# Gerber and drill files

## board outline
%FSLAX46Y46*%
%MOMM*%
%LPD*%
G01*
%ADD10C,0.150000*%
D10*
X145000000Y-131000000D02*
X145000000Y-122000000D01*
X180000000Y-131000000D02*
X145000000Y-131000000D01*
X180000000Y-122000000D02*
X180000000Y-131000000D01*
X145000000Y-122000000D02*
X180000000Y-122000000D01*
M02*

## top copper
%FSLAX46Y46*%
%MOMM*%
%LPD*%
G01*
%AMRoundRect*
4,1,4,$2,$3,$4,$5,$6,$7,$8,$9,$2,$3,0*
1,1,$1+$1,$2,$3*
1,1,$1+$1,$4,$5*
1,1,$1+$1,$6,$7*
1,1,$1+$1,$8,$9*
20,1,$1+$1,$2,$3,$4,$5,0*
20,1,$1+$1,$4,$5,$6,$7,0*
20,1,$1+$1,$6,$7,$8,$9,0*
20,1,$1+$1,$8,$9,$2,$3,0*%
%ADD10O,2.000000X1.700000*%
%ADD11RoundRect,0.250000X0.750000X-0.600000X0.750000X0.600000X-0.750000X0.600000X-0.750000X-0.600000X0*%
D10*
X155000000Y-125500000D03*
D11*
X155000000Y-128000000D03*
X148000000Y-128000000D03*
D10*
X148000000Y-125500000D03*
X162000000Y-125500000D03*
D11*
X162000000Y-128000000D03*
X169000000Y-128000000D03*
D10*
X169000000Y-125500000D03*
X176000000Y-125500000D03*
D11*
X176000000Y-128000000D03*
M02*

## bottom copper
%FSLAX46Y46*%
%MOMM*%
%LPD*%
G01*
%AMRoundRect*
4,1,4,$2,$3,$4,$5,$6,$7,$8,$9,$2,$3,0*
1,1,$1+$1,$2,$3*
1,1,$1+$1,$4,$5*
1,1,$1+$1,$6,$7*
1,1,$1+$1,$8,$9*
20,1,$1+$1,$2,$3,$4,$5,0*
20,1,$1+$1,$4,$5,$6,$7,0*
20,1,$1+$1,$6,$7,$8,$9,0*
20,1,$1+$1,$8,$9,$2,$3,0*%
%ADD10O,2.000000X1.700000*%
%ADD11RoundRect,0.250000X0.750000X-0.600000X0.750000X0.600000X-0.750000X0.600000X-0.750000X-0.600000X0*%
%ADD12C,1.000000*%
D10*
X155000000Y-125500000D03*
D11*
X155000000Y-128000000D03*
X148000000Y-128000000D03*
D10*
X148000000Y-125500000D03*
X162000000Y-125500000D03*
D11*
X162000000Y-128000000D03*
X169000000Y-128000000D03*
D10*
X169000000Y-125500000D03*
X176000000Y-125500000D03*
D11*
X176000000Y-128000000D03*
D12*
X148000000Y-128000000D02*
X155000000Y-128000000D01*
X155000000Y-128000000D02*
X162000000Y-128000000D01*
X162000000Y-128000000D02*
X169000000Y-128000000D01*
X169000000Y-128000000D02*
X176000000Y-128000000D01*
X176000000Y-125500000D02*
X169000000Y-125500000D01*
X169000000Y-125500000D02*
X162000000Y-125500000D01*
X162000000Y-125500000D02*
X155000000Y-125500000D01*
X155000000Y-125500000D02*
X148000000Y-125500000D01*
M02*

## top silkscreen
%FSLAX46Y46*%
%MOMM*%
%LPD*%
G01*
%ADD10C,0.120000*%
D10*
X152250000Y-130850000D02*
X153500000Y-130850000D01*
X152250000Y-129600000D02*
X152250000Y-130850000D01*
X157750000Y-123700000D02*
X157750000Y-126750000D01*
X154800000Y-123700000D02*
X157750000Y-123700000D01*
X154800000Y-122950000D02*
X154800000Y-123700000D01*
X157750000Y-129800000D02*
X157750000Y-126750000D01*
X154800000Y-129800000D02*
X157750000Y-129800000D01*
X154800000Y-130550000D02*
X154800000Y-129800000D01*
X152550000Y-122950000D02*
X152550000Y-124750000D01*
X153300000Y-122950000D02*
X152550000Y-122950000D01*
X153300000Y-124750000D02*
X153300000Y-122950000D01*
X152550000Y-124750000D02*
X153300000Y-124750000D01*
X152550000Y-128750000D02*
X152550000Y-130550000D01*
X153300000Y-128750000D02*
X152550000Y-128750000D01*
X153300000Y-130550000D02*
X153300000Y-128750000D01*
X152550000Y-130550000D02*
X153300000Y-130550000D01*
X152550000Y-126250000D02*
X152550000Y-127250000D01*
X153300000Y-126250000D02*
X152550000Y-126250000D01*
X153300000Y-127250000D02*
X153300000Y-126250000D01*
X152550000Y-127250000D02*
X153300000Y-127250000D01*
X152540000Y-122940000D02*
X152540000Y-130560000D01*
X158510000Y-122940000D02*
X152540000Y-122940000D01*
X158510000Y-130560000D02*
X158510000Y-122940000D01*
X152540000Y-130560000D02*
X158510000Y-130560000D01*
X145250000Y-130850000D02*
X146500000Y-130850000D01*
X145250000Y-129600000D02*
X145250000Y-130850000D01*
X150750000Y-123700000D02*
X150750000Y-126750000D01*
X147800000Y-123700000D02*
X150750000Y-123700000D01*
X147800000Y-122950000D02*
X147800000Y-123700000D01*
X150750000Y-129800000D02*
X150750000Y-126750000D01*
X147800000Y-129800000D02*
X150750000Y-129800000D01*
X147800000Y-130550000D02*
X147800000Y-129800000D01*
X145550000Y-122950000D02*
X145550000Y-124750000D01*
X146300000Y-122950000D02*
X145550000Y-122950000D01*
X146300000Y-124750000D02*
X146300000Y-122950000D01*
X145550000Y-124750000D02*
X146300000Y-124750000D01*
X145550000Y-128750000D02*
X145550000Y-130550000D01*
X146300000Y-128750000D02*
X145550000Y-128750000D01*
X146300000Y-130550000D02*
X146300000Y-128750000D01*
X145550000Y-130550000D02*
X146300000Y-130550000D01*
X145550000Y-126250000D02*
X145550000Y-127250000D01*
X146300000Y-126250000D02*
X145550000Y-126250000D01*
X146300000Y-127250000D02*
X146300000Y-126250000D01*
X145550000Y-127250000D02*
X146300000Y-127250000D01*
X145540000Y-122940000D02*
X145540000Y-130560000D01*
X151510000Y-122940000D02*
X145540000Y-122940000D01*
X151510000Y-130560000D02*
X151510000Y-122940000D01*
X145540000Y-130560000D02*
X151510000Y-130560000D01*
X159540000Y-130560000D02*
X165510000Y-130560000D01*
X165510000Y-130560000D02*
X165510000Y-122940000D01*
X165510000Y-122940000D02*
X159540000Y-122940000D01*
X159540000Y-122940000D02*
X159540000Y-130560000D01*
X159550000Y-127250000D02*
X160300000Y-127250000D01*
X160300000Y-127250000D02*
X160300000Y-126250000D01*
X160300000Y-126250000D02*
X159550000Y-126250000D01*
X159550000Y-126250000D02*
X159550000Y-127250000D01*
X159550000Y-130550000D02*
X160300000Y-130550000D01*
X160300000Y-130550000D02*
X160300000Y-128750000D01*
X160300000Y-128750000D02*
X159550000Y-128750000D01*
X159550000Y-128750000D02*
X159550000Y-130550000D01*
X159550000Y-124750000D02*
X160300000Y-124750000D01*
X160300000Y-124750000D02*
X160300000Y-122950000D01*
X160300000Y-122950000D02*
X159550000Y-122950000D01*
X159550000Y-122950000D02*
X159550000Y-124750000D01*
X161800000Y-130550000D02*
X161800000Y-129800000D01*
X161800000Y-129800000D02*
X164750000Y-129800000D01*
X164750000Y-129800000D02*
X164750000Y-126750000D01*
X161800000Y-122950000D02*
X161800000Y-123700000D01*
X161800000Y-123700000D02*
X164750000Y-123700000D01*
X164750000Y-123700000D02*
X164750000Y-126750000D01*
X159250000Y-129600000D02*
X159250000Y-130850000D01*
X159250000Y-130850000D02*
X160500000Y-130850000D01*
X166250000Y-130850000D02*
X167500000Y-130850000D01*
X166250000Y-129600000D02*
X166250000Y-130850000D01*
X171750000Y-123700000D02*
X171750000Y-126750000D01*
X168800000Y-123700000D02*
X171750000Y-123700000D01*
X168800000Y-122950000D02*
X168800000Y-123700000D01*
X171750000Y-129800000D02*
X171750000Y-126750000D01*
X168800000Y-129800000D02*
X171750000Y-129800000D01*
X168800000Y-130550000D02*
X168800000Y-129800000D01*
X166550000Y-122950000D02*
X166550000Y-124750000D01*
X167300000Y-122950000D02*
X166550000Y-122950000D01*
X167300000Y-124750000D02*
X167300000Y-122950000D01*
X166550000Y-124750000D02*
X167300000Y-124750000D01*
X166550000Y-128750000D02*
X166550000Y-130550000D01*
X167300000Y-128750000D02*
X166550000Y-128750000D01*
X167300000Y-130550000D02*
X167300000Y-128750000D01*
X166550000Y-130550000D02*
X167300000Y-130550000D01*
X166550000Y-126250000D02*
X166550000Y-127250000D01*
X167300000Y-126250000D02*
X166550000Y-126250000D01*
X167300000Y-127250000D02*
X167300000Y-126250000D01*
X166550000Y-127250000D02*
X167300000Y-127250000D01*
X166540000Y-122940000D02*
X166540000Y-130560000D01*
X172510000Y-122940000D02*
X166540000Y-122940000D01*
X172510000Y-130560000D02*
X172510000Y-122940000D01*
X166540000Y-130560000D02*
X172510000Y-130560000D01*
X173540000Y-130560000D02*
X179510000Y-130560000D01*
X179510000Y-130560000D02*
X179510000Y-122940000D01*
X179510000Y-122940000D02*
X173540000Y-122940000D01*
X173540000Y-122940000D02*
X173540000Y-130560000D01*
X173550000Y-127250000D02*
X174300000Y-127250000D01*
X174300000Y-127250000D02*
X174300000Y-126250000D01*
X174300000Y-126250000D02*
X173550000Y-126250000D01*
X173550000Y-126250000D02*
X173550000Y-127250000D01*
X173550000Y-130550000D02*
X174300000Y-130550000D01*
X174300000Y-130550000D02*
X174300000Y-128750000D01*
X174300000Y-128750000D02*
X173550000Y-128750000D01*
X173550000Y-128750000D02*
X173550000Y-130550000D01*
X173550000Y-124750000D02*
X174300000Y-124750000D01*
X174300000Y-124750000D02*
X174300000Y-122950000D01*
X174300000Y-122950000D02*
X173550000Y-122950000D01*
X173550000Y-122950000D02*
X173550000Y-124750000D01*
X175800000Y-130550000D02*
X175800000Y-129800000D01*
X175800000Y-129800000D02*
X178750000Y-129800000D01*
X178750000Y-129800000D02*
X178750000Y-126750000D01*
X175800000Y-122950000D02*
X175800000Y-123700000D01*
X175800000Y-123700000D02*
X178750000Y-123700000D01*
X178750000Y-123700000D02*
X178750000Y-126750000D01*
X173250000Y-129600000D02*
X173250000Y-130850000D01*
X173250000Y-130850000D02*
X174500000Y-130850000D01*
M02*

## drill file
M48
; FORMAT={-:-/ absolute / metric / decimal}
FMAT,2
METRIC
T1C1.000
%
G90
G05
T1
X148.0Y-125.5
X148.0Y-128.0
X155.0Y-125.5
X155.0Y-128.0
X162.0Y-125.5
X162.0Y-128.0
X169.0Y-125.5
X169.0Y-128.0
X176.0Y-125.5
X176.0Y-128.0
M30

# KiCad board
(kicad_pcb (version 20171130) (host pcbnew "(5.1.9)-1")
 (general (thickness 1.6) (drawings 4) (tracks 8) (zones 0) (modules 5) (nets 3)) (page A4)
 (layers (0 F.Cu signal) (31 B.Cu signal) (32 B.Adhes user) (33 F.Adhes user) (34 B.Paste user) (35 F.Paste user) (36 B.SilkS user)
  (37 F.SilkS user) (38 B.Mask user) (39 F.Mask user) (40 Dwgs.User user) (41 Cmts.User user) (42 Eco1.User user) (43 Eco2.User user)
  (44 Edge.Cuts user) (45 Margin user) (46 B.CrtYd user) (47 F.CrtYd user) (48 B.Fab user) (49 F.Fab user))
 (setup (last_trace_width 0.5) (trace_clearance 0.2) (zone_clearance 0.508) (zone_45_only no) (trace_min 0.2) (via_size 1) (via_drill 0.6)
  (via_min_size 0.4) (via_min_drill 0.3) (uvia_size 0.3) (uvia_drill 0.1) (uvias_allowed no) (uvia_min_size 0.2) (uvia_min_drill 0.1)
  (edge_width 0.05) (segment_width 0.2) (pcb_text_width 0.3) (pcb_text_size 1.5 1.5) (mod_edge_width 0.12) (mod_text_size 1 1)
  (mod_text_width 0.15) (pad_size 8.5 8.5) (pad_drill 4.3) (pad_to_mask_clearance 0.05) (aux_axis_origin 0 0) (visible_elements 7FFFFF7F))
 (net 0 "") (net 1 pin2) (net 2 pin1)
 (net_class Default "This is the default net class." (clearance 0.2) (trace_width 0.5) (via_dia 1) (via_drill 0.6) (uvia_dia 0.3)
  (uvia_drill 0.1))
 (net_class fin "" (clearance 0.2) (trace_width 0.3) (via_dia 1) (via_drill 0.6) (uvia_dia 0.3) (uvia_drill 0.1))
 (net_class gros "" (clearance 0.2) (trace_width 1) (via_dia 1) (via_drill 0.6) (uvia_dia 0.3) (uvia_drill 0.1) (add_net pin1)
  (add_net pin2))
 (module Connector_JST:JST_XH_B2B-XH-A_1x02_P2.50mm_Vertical (layer F.Cu) (at 155 128 90)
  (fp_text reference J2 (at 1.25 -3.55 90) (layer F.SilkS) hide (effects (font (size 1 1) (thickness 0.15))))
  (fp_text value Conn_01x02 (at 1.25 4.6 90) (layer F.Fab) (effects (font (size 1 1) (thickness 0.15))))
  (fp_line (start -2.85 -2.75) (end -2.85 -1.5) (layer F.SilkS) (width 0.12))
  (fp_line (start -1.6 -2.75) (end -2.85 -2.75) (layer F.SilkS) (width 0.12))
  (fp_line (start 4.3 2.75) (end 1.25 2.75) (layer F.SilkS) (width 0.12))
  (fp_line (start 4.3 -0.2) (end 4.3 2.75) (layer F.SilkS) (width 0.12))
  (fp_line (start 5.05 -0.2) (end 4.3 -0.2) (layer F.SilkS) (width 0.12))
  (fp_line (start -1.8 2.75) (end 1.25 2.75) (layer F.SilkS) (width 0.12))
  (fp_line (start -1.8 -0.2) (end -1.8 2.75) (layer F.SilkS) (width 0.12))
  (fp_line (start -2.55 -0.2) (end -1.8 -0.2) (layer F.SilkS) (width 0.12))
  (fp_line (start 5.05 -2.45) (end 3.25 -2.45) (layer F.SilkS) (width 0.12))
  (fp_line (start 5.05 -1.7) (end 5.05 -2.45) (layer F.SilkS) (width 0.12))
  (fp_line (start 3.25 -1.7) (end 5.05 -1.7) (layer F.SilkS) (width 0.12))
  (fp_line (start 3.25 -2.45) (end 3.25 -1.7) (layer F.SilkS) (width 0.12))
  (fp_line (start -0.75 -2.45) (end -2.55 -2.45) (layer F.SilkS) (width 0.12))
  (fp_line (start -0.75 -1.7) (end -0.75 -2.45) (layer F.SilkS) (width 0.12))
  (fp_line (start -2.55 -1.7) (end -0.75 -1.7) (layer F.SilkS) (width 0.12))
  (fp_line (start -2.55 -2.45) (end -2.55 -1.7) (layer F.SilkS) (width 0.12))
  (fp_line (start 1.75 -2.45) (end 0.75 -2.45) (layer F.SilkS) (width 0.12))
  (fp_line (start 1.75 -1.7) (end 1.75 -2.45) (layer F.SilkS) (width 0.12))
  (fp_line (start 0.75 -1.7) (end 1.75 -1.7) (layer F.SilkS) (width 0.12))
  (fp_line (start 0.75 -2.45) (end 0.75 -1.7) (layer F.SilkS) (width 0.12))
  (fp_line (start 5.06 -2.46) (end -2.56 -2.46) (layer F.SilkS) (width 0.12))
  (fp_line (start 5.06 3.51) (end 5.06 -2.46) (layer F.SilkS) (width 0.12))
  (fp_line (start -2.56 3.51) (end 5.06 3.51) (layer F.SilkS) (width 0.12))
  (fp_line (start -2.56 -2.46) (end -2.56 3.51) (layer F.SilkS) (width 0.12))
  (pad 2 thru_hole oval (at 2.5 0 90) (size 1.7 2) (drill 1) (layers *.Cu *.Mask) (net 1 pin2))
  (pad 1 thru_hole roundrect (at 0 0 90) (size 1.7 2) (drill 1) (layers *.Cu *.Mask) (roundrect_rratio 0.147059) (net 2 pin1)))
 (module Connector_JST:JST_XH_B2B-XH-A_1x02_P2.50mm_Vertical (layer F.Cu) (at 148 128 90)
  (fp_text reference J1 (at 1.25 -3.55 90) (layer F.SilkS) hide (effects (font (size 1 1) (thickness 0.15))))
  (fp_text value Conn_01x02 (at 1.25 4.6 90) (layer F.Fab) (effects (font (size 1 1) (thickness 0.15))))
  (fp_line (start -2.85 -2.75) (end -2.85 -1.5) (layer F.SilkS) (width 0.12))
  (fp_line (start -1.6 -2.75) (end -2.85 -2.75) (layer F.SilkS) (width 0.12))
  (fp_line (start 4.3 2.75) (end 1.25 2.75) (layer F.SilkS) (width 0.12))
  (fp_line (start 4.3 -0.2) (end 4.3 2.75) (layer F.SilkS) (width 0.12))
  (fp_line (start 5.05 -0.2) (end 4.3 -0.2) (layer F.SilkS) (width 0.12))
  (fp_line (start -1.8 2.75) (end 1.25 2.75) (layer F.SilkS) (width 0.12))
  (fp_line (start -1.8 -0.2) (end -1.8 2.75) (layer F.SilkS) (width 0.12))
  (fp_line (start -2.55 -0.2) (end -1.8 -0.2) (layer F.SilkS) (width 0.12))
  (fp_line (start 5.05 -2.45) (end 3.25 -2.45) (layer F.SilkS) (width 0.12))
  (fp_line (start 5.05 -1.7) (end 5.05 -2.45) (layer F.SilkS) (width 0.12))
  (fp_line (start 3.25 -1.7) (end 5.05 -1.7) (layer F.SilkS) (width 0.12))
  (fp_line (start 3.25 -2.45) (end 3.25 -1.7) (layer F.SilkS) (width 0.12))
  (fp_line (start -0.75 -2.45) (end -2.55 -2.45) (layer F.SilkS) (width 0.12))
  (fp_line (start -0.75 -1.7) (end -0.75 -2.45) (layer F.SilkS) (width 0.12))
  (fp_line (start -2.55 -1.7) (end -0.75 -1.7) (layer F.SilkS) (width 0.12))
  (fp_line (start -2.55 -2.45) (end -2.55 -1.7) (layer F.SilkS) (width 0.12))
  (fp_line (start 1.75 -2.45) (end 0.75 -2.45) (layer F.SilkS) (width 0.12))
  (fp_line (start 1.75 -1.7) (end 1.75 -2.45) (layer F.SilkS) (width 0.12))
  (fp_line (start 0.75 -1.7) (end 1.75 -1.7) (layer F.SilkS) (width 0.12))
  (fp_line (start 0.75 -2.45) (end 0.75 -1.7) (layer F.SilkS) (width 0.12))
  (fp_line (start 5.06 -2.46) (end -2.56 -2.46) (layer F.SilkS) (width 0.12))
  (fp_line (start 5.06 3.51) (end 5.06 -2.46) (layer F.SilkS) (width 0.12))
  (fp_line (start -2.56 3.51) (end 5.06 3.51) (layer F.SilkS) (width 0.12))
  (fp_line (start -2.56 -2.46) (end -2.56 3.51) (layer F.SilkS) (width 0.12))
  (pad 1 thru_hole roundrect (at 0 0 90) (size 1.7 2) (drill 1) (layers *.Cu *.Mask) (roundrect_rratio 0.147059) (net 2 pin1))
  (pad 2 thru_hole oval (at 2.5 0 90) (size 1.7 2) (drill 1) (layers *.Cu *.Mask) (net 1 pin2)))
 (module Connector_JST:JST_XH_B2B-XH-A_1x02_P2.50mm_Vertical (layer F.Cu) (at 162 128 90)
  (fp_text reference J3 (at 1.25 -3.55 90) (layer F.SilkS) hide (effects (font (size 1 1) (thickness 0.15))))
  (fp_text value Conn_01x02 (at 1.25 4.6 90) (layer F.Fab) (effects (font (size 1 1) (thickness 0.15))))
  (fp_line (start -2.56 -2.46) (end -2.56 3.51) (layer F.SilkS) (width 0.12))
  (fp_line (start -2.56 3.51) (end 5.06 3.51) (layer F.SilkS) (width 0.12))
  (fp_line (start 5.06 3.51) (end 5.06 -2.46) (layer F.SilkS) (width 0.12))
  (fp_line (start 5.06 -2.46) (end -2.56 -2.46) (layer F.SilkS) (width 0.12))
  (fp_line (start 0.75 -2.45) (end 0.75 -1.7) (layer F.SilkS) (width 0.12))
  (fp_line (start 0.75 -1.7) (end 1.75 -1.7) (layer F.SilkS) (width 0.12))
  (fp_line (start 1.75 -1.7) (end 1.75 -2.45) (layer F.SilkS) (width 0.12))
  (fp_line (start 1.75 -2.45) (end 0.75 -2.45) (layer F.SilkS) (width 0.12))
  (fp_line (start -2.55 -2.45) (end -2.55 -1.7) (layer F.SilkS) (width 0.12))
  (fp_line (start -2.55 -1.7) (end -0.75 -1.7) (layer F.SilkS) (width 0.12))
  (fp_line (start -0.75 -1.7) (end -0.75 -2.45) (layer F.SilkS) (width 0.12))
  (fp_line (start -0.75 -2.45) (end -2.55 -2.45) (layer F.SilkS) (width 0.12))
  (fp_line (start 3.25 -2.45) (end 3.25 -1.7) (layer F.SilkS) (width 0.12))
  (fp_line (start 3.25 -1.7) (end 5.05 -1.7) (layer F.SilkS) (width 0.12))
  (fp_line (start 5.05 -1.7) (end 5.05 -2.45) (layer F.SilkS) (width 0.12))
  (fp_line (start 5.05 -2.45) (end 3.25 -2.45) (layer F.SilkS) (width 0.12))
  (fp_line (start -2.55 -0.2) (end -1.8 -0.2) (layer F.SilkS) (width 0.12))
  (fp_line (start -1.8 -0.2) (end -1.8 2.75) (layer F.SilkS) (width 0.12))
  (fp_line (start -1.8 2.75) (end 1.25 2.75) (layer F.SilkS) (width 0.12))
  (fp_line (start 5.05 -0.2) (end 4.3 -0.2) (layer F.SilkS) (width 0.12))
  (fp_line (start 4.3 -0.2) (end 4.3 2.75) (layer F.SilkS) (width 0.12))
  (fp_line (start 4.3 2.75) (end 1.25 2.75) (layer F.SilkS) (width 0.12))
  (fp_line (start -1.6 -2.75) (end -2.85 -2.75) (layer F.SilkS) (width 0.12))
  (fp_line (start -2.85 -2.75) (end -2.85 -1.5) (layer F.SilkS) (width 0.12))
  (pad 2 thru_hole oval (at 2.5 0 90) (size 1.7 2) (drill 1) (layers *.Cu *.Mask) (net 1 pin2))
  (pad 1 thru_hole roundrect (at 0 0 90) (size 1.7 2) (drill 1) (layers *.Cu *.Mask) (roundrect_rratio 0.147059) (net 2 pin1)))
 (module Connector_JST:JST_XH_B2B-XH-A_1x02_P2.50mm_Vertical (layer F.Cu) (at 169 128 90)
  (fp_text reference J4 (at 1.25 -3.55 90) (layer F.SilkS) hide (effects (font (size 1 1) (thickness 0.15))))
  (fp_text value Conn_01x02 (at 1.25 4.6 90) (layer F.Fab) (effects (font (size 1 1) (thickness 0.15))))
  (fp_line (start -2.85 -2.75) (end -2.85 -1.5) (layer F.SilkS) (width 0.12))
  (fp_line (start -1.6 -2.75) (end -2.85 -2.75) (layer F.SilkS) (width 0.12))
  (fp_line (start 4.3 2.75) (end 1.25 2.75) (layer F.SilkS) (width 0.12))
  (fp_line (start 4.3 -0.2) (end 4.3 2.75) (layer F.SilkS) (width 0.12))
  (fp_line (start 5.05 -0.2) (end 4.3 -0.2) (layer F.SilkS) (width 0.12))
  (fp_line (start -1.8 2.75) (end 1.25 2.75) (layer F.SilkS) (width 0.12))
  (fp_line (start -1.8 -0.2) (end -1.8 2.75) (layer F.SilkS) (width 0.12))
  (fp_line (start -2.55 -0.2) (end -1.8 -0.2) (layer F.SilkS) (width 0.12))
  (fp_line (start 5.05 -2.45) (end 3.25 -2.45) (layer F.SilkS) (width 0.12))
  (fp_line (start 5.05 -1.7) (end 5.05 -2.45) (layer F.SilkS) (width 0.12))
  (fp_line (start 3.25 -1.7) (end 5.05 -1.7) (layer F.SilkS) (width 0.12))
  (fp_line (start 3.25 -2.45) (end 3.25 -1.7) (layer F.SilkS) (width 0.12))
  (fp_line (start -0.75 -2.45) (end -2.55 -2.45) (layer F.SilkS) (width 0.12))
  (fp_line (start -0.75 -1.7) (end -0.75 -2.45) (layer F.SilkS) (width 0.12))
  (fp_line (start -2.55 -1.7) (end -0.75 -1.7) (layer F.SilkS) (width 0.12))
  (fp_line (start -2.55 -2.45) (end -2.55 -1.7) (layer F.SilkS) (width 0.12))
  (fp_line (start 1.75 -2.45) (end 0.75 -2.45) (layer F.SilkS) (width 0.12))
  (fp_line (start 1.75 -1.7) (end 1.75 -2.45) (layer F.SilkS) (width 0.12))
  (fp_line (start 0.75 -1.7) (end 1.75 -1.7) (layer F.SilkS) (width 0.12))
  (fp_line (start 0.75 -2.45) (end 0.75 -1.7) (layer F.SilkS) (width 0.12))
  (fp_line (start 5.06 -2.46) (end -2.56 -2.46) (layer F.SilkS) (width 0.12))
  (fp_line (start 5.06 3.51) (end 5.06 -2.46) (layer F.SilkS) (width 0.12))
  (fp_line (start -2.56 3.51) (end 5.06 3.51) (layer F.SilkS) (width 0.12))
  (fp_line (start -2.56 -2.46) (end -2.56 3.51) (layer F.SilkS) (width 0.12))
  (pad 1 thru_hole roundrect (at 0 0 90) (size 1.7 2) (drill 1) (layers *.Cu *.Mask) (roundrect_rratio 0.147059) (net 2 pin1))
  (pad 2 thru_hole oval (at 2.5 0 90) (size 1.7 2) (drill 1) (layers *.Cu *.Mask) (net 1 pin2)))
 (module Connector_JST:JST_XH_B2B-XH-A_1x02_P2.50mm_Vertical (layer F.Cu) (at 176 128 90)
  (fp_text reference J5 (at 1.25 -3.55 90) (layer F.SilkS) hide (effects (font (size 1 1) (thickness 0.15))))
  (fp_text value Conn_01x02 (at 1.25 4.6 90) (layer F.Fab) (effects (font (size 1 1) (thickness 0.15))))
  (fp_line (start -2.56 -2.46) (end -2.56 3.51) (layer F.SilkS) (width 0.12))
  (fp_line (start -2.56 3.51) (end 5.06 3.51) (layer F.SilkS) (width 0.12))
  (fp_line (start 5.06 3.51) (end 5.06 -2.46) (layer F.SilkS) (width 0.12))
  (fp_line (start 5.06 -2.46) (end -2.56 -2.46) (layer F.SilkS) (width 0.12))
  (fp_line (start 0.75 -2.45) (end 0.75 -1.7) (layer F.SilkS) (width 0.12))
  (fp_line (start 0.75 -1.7) (end 1.75 -1.7) (layer F.SilkS) (width 0.12))
  (fp_line (start 1.75 -1.7) (end 1.75 -2.45) (layer F.SilkS) (width 0.12))
  (fp_line (start 1.75 -2.45) (end 0.75 -2.45) (layer F.SilkS) (width 0.12))
  (fp_line (start -2.55 -2.45) (end -2.55 -1.7) (layer F.SilkS) (width 0.12))
  (fp_line (start -2.55 -1.7) (end -0.75 -1.7) (layer F.SilkS) (width 0.12))
  (fp_line (start -0.75 -1.7) (end -0.75 -2.45) (layer F.SilkS) (width 0.12))
  (fp_line (start -0.75 -2.45) (end -2.55 -2.45) (layer F.SilkS) (width 0.12))
  (fp_line (start 3.25 -2.45) (end 3.25 -1.7) (layer F.SilkS) (width 0.12))
  (fp_line (start 3.25 -1.7) (end 5.05 -1.7) (layer F.SilkS) (width 0.12))
  (fp_line (start 5.05 -1.7) (end 5.05 -2.45) (layer F.SilkS) (width 0.12))
  (fp_line (start 5.05 -2.45) (end 3.25 -2.45) (layer F.SilkS) (width 0.12))
  (fp_line (start -2.55 -0.2) (end -1.8 -0.2) (layer F.SilkS) (width 0.12))
  (fp_line (start -1.8 -0.2) (end -1.8 2.75) (layer F.SilkS) (width 0.12))
  (fp_line (start -1.8 2.75) (end 1.25 2.75) (layer F.SilkS) (width 0.12))
  (fp_line (start 5.05 -0.2) (end 4.3 -0.2) (layer F.SilkS) (width 0.12))
  (fp_line (start 4.3 -0.2) (end 4.3 2.75) (layer F.SilkS) (width 0.12))
  (fp_line (start 4.3 2.75) (end 1.25 2.75) (layer F.SilkS) (width 0.12))
  (fp_line (start -1.6 -2.75) (end -2.85 -2.75) (layer F.SilkS) (width 0.12))
  (fp_line (start -2.85 -2.75) (end -2.85 -1.5) (layer F.SilkS) (width 0.12))
  (pad 2 thru_hole oval (at 2.5 0 90) (size 1.7 2) (drill 1) (layers *.Cu *.Mask) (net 1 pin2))
  (pad 1 thru_hole roundrect (at 0 0 90) (size 1.7 2) (drill 1) (layers *.Cu *.Mask) (roundrect_rratio 0.147059) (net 2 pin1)))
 (gr_line (start 145 131) (end 145 122) (layer Edge.Cuts) (width 0.15))
 (gr_line (start 180 131) (end 145 131) (layer Edge.Cuts) (width 0.15))
 (gr_line (start 180 122) (end 180 131) (layer Edge.Cuts) (width 0.15))
 (gr_line (start 145 122) (end 180 122) (layer Edge.Cuts) (width 0.15))
 (segment (start 148 128) (end 155 128) (width 1) (layer B.Cu) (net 2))
 (segment (start 155 128) (end 162 128) (width 1) (layer B.Cu) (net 2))
 (segment (start 162 128) (end 169 128) (width 1) (layer B.Cu) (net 2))
 (segment (start 169 128) (end 176 128) (width 1) (layer B.Cu) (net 2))
 (segment (start 176 125.5) (end 169 125.5) (width 1) (layer B.Cu) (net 1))
 (segment (start 169 125.5) (end 162 125.5) (width 1) (layer B.Cu) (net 1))
 (segment (start 162 125.5) (end 155 125.5) (width 1) (layer B.Cu) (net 1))
 (segment (start 155 125.5) (end 148 125.5) (width 1) (layer B.Cu) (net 1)))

